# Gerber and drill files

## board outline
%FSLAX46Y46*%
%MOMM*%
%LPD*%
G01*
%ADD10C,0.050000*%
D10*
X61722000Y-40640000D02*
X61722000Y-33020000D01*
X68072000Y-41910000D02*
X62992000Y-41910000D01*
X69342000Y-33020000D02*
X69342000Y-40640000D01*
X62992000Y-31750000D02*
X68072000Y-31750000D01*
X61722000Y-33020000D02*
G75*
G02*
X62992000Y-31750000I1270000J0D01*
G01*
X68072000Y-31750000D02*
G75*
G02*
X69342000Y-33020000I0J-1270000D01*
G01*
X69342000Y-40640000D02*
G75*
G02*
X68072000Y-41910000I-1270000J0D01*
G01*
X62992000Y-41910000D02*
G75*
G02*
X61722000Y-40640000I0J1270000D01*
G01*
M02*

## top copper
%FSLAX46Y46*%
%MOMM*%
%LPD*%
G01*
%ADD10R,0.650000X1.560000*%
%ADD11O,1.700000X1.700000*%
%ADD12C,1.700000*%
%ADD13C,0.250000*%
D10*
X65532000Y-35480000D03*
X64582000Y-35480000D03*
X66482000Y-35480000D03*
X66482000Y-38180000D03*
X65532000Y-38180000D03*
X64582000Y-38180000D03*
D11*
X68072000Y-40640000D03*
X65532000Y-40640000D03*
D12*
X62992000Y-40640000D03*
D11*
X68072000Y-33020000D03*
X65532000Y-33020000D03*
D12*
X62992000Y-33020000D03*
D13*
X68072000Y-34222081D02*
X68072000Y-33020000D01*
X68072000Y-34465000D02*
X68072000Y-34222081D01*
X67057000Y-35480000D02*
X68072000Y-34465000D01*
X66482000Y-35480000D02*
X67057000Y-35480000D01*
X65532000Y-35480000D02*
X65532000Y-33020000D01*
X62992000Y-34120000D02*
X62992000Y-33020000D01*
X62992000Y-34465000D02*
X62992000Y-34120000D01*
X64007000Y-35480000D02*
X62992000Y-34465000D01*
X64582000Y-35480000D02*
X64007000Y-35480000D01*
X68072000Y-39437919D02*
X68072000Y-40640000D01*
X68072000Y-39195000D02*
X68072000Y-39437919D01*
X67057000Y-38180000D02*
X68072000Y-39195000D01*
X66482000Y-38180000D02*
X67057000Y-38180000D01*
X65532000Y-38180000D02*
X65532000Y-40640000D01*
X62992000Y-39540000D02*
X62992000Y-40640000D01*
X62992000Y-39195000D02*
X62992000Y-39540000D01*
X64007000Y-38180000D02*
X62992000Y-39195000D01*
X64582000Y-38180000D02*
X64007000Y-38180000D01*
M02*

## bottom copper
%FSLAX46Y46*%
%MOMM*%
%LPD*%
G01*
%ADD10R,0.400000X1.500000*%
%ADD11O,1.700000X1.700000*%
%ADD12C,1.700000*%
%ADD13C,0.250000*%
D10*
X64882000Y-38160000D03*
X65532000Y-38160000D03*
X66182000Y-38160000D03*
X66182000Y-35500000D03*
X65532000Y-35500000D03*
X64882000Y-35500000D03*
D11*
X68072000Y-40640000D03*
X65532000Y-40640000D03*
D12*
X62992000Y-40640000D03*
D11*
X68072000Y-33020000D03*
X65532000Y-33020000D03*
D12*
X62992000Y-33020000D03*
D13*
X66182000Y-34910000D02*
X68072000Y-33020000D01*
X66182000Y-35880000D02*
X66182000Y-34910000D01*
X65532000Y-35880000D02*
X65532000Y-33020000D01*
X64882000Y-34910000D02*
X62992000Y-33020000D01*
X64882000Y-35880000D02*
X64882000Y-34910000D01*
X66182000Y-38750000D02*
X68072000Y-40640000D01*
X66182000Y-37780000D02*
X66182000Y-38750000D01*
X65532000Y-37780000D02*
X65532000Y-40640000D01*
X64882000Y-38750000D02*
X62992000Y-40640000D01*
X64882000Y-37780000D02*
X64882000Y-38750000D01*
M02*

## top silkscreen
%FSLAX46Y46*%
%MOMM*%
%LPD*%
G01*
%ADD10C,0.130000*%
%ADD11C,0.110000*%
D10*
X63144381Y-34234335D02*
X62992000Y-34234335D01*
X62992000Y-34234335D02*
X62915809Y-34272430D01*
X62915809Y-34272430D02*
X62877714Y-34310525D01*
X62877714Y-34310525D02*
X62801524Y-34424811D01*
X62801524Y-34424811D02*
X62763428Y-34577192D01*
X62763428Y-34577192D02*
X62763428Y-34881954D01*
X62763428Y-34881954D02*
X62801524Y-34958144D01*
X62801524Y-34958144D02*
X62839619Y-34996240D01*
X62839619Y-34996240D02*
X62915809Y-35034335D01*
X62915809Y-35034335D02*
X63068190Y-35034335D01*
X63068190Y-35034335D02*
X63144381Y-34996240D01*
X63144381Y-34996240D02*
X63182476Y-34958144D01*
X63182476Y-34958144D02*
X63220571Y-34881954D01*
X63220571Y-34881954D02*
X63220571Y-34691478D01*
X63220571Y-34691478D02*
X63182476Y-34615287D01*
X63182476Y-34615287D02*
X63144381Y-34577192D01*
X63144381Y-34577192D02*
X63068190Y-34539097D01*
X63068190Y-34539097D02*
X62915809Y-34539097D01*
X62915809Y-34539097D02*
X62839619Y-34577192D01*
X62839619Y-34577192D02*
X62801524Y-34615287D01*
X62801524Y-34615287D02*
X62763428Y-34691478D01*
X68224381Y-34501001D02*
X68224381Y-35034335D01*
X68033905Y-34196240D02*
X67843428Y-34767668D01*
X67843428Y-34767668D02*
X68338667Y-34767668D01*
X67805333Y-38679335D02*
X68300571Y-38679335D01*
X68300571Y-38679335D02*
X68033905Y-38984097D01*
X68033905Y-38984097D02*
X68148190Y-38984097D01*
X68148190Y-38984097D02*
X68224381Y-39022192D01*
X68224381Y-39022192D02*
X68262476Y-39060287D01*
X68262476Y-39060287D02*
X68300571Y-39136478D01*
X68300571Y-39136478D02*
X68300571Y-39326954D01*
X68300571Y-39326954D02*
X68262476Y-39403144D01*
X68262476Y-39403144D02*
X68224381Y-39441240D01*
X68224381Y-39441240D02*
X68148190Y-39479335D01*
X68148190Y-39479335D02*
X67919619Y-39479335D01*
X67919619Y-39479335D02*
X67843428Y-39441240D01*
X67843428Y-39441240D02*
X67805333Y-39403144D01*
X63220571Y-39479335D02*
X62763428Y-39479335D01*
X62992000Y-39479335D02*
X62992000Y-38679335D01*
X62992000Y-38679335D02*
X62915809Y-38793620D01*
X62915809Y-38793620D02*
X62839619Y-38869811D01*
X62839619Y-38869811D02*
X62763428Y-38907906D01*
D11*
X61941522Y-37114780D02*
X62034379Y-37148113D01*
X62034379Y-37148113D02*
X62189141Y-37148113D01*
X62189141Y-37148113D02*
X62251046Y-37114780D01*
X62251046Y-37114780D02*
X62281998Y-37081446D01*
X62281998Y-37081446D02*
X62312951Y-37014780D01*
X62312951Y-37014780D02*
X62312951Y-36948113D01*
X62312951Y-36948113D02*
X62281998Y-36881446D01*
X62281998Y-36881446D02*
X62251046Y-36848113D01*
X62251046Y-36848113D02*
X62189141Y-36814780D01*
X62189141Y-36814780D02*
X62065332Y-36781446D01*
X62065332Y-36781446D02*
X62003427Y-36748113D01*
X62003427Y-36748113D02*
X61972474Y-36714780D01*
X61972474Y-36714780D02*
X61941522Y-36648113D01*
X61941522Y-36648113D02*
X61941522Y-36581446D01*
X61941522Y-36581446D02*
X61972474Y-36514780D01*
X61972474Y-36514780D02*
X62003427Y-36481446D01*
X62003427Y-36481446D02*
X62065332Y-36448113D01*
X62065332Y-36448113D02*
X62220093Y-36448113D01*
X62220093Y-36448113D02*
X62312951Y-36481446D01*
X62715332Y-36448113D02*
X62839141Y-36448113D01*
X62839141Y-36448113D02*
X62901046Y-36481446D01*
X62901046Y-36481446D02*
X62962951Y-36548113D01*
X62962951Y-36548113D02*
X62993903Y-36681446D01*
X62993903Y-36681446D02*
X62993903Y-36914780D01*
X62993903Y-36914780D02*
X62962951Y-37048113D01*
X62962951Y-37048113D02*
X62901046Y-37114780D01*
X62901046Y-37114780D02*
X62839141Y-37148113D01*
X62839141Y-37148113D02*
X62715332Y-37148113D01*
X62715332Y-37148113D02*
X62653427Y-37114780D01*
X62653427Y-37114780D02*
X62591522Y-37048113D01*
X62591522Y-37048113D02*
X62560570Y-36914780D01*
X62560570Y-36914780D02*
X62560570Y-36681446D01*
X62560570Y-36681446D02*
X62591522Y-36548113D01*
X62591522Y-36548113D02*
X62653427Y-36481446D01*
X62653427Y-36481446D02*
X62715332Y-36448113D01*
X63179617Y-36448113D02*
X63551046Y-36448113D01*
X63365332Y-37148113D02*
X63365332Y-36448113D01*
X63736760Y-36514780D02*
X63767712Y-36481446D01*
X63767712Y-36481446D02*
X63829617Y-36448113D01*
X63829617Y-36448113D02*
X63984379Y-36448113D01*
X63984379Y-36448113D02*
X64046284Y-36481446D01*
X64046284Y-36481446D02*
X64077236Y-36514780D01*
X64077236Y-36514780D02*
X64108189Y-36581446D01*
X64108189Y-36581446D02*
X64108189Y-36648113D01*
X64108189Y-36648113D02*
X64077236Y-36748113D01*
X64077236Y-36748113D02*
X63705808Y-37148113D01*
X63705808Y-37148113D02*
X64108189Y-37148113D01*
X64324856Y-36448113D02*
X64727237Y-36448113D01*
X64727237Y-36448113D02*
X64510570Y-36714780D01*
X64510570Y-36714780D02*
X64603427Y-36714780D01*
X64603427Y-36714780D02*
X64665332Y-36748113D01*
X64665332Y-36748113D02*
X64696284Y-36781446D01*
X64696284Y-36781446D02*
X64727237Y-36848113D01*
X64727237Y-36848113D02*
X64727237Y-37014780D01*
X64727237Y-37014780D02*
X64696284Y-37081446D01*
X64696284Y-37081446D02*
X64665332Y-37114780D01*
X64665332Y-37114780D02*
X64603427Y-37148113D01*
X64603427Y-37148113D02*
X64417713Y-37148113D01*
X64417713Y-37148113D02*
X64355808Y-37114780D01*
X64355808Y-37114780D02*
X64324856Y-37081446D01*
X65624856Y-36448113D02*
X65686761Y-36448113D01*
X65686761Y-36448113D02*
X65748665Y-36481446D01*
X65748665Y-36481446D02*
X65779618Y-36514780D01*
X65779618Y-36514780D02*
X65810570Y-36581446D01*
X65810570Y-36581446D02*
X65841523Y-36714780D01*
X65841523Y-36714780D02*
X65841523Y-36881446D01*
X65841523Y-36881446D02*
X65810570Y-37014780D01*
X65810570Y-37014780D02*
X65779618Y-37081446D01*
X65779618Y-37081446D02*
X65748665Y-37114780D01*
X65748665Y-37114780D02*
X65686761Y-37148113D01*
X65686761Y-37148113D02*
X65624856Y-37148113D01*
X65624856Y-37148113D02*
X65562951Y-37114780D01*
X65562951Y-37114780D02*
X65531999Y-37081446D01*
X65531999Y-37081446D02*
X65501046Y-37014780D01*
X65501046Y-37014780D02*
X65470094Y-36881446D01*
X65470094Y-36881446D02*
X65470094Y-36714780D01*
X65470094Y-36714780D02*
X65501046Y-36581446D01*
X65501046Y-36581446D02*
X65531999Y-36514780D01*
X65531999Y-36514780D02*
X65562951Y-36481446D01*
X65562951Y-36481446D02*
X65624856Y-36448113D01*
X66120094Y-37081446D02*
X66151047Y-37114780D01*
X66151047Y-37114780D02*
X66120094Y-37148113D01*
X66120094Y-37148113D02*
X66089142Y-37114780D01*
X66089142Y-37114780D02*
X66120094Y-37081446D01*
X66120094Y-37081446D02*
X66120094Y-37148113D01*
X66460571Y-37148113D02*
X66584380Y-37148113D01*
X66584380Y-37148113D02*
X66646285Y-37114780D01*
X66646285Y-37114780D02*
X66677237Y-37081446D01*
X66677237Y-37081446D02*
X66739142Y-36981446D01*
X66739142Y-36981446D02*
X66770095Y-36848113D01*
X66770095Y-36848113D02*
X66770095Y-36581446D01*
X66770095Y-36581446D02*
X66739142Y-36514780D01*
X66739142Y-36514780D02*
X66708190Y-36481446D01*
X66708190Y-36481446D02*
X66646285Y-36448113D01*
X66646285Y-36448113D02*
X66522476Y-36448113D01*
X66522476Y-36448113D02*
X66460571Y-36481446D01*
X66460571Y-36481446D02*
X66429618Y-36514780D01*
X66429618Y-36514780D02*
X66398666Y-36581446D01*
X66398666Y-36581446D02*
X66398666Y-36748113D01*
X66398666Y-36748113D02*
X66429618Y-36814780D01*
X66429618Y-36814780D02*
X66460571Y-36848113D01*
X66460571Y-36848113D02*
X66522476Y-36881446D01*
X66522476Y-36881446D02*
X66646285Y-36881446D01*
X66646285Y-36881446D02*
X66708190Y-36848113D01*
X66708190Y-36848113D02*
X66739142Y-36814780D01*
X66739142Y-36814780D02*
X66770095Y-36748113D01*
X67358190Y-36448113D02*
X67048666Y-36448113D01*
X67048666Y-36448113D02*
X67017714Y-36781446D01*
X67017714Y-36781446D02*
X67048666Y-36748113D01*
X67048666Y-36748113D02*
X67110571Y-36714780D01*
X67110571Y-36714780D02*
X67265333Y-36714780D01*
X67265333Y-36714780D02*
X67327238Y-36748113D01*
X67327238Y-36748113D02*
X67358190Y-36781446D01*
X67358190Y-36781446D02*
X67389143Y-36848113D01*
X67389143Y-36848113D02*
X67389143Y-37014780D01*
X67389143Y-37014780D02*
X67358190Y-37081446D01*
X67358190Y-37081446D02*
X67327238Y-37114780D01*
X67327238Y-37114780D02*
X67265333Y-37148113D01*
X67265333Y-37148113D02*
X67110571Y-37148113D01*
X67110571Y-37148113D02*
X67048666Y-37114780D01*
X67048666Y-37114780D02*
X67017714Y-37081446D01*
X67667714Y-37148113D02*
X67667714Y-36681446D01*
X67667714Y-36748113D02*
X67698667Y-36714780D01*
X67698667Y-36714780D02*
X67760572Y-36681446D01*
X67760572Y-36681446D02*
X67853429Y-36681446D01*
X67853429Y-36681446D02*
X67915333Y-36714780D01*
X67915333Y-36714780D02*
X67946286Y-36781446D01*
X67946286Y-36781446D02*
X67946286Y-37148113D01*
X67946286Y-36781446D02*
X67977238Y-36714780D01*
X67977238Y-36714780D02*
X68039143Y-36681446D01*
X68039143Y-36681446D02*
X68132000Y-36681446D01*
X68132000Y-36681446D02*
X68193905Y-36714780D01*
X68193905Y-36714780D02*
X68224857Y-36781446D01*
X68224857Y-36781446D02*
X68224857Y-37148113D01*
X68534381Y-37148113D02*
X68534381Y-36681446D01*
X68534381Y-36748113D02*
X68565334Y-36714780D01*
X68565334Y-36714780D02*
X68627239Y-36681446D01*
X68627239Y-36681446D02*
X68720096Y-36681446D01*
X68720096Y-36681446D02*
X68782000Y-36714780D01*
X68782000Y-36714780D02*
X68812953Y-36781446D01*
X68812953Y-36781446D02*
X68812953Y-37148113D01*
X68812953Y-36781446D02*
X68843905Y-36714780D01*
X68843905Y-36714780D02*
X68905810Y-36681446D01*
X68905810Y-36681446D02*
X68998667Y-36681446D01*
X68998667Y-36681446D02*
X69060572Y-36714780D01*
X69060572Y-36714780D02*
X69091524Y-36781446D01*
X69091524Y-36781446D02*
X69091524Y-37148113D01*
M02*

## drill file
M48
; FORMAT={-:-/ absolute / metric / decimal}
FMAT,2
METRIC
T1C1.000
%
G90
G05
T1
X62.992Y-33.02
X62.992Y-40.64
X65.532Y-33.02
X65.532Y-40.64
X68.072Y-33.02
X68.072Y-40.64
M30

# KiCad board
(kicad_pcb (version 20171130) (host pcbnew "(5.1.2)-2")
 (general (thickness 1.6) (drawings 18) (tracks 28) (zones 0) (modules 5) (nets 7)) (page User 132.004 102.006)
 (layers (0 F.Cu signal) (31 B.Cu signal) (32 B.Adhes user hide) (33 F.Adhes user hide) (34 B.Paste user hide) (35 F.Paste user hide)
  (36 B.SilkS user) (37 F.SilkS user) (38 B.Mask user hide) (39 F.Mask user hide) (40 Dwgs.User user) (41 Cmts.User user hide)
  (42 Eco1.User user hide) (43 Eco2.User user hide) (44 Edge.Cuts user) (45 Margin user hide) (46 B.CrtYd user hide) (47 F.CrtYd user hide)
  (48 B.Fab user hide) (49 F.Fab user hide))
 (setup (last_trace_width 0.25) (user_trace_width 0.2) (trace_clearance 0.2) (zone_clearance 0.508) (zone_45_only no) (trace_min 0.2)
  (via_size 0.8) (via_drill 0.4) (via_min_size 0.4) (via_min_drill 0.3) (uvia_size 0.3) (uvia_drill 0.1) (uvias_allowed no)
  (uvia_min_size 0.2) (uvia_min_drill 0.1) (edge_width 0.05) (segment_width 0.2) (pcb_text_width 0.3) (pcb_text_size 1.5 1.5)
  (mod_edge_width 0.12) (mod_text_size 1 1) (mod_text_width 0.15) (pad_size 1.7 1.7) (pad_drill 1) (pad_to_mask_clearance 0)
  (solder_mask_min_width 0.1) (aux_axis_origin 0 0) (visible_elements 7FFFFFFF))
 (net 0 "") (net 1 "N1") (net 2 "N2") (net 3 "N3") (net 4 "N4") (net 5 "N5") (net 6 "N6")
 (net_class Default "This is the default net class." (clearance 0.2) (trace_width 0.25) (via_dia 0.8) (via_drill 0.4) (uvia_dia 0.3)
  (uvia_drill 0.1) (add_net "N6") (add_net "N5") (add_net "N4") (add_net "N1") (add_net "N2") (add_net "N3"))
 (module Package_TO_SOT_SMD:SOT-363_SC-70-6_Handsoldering (layer B.Cu) (at 65.532 36.83 270)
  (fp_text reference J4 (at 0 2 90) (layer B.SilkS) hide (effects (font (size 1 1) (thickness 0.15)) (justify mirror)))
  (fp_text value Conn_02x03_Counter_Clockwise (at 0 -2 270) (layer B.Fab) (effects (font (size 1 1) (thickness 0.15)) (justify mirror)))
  (pad 6 smd rect (at 1.33 0.65 270) (size 1.5 0.4) (layers B.Cu B.Paste B.Mask) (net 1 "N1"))
  (pad 5 smd rect (at 1.33 0 270) (size 1.5 0.4) (layers B.Cu B.Paste B.Mask) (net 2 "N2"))
  (pad 4 smd rect (at 1.33 -0.65 270) (size 1.5 0.4) (layers B.Cu B.Paste B.Mask) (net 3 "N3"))
  (pad 3 smd rect (at -1.33 -0.65 270) (size 1.5 0.4) (layers B.Cu B.Paste B.Mask) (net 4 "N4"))
  (pad 2 smd rect (at -1.33 0 270) (size 1.5 0.4) (layers B.Cu B.Paste B.Mask) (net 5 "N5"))
  (pad 1 smd rect (at -1.33 0.65 270) (size 1.5 0.4) (layers B.Cu B.Paste B.Mask) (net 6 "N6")))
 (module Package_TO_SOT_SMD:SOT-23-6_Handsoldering (layer F.Cu) (at 65.532 36.83 90)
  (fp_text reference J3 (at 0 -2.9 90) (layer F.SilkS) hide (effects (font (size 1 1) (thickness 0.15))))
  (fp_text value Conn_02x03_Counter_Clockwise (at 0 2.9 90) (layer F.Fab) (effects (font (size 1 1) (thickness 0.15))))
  (pad 5 smd rect (at 1.35 0 90) (size 1.56 0.65) (layers F.Cu F.Paste F.Mask) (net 5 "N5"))
  (pad 6 smd rect (at 1.35 -0.95 90) (size 1.56 0.65) (layers F.Cu F.Paste F.Mask) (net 6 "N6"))
  (pad 4 smd rect (at 1.35 0.95 90) (size 1.56 0.65) (layers F.Cu F.Paste F.Mask) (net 4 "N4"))
  (pad 3 smd rect (at -1.35 0.95 90) (size 1.56 0.65) (layers F.Cu F.Paste F.Mask) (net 3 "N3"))
  (pad 2 smd rect (at -1.35 0 90) (size 1.56 0.65) (layers F.Cu F.Paste F.Mask) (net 2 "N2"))
  (pad 1 smd rect (at -1.35 -0.95 90) (size 1.56 0.65) (layers F.Cu F.Paste F.Mask) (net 1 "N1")))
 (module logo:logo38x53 (layer B.Cu) (at 62.992 36.8046 180)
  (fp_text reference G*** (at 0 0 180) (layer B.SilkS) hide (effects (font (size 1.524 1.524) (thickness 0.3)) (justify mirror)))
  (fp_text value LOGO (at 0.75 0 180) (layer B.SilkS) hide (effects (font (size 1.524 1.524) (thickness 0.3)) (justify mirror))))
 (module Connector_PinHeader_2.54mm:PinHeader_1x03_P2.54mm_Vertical (layer F.Cu) (at 62.992 40.64 90)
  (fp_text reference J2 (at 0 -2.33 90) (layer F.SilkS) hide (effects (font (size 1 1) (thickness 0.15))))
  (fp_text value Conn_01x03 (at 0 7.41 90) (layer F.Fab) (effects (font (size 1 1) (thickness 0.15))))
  (pad 3 thru_hole oval (at 0 5.08 90) (size 1.7 1.7) (drill 1) (layers *.Cu *.Mask) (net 3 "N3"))
  (pad 2 thru_hole oval (at 0 2.54 90) (size 1.7 1.7) (drill 1) (layers *.Cu *.Mask) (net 2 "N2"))
  (pad 1 thru_hole circle (at 0 0 90) (size 1.7 1.7) (drill 1) (layers *.Cu *.Mask) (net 1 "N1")))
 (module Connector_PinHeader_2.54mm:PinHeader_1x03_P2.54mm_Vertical (layer F.Cu) (at 62.992 33.02 90)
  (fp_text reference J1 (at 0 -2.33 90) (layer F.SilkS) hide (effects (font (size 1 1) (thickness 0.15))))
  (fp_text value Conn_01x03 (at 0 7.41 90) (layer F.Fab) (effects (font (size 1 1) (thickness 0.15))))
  (pad 3 thru_hole oval (at 0 5.08 90) (size 1.7 1.7) (drill 1) (layers *.Cu *.Mask) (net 4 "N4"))
  (pad 2 thru_hole oval (at 0 2.54 90) (size 1.7 1.7) (drill 1) (layers *.Cu *.Mask) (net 5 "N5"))
  (pad 1 thru_hole circle (at 0 0 90) (size 1.7 1.7) (drill 1) (layers *.Cu *.Mask) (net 6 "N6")))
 (gr_line (start 61.722 40.64) (end 61.722 33.02) (layer Edge.Cuts) (width 0.05))
 (gr_line (start 68.072 41.91) (end 62.992 41.91) (layer Edge.Cuts) (width 0.05))
 (gr_line (start 69.342 33.02) (end 69.342 40.64) (layer Edge.Cuts) (width 0.05))
 (gr_line (start 62.992 31.75) (end 68.072 31.75) (layer Edge.Cuts) (width 0.05))
 (gr_arc (start 62.992 33.02) (end 62.992 31.75) (angle -90) (layer Edge.Cuts) (width 0.05))
 (gr_arc (start 68.072 33.02) (end 69.342 33.02) (angle -90) (layer Edge.Cuts) (width 0.05))
 (gr_arc (start 68.072 40.64) (end 68.072 41.91) (angle -90) (layer Edge.Cuts) (width 0.05))
 (gr_arc (start 62.992 40.64) (end 61.722 40.64) (angle -90) (layer Edge.Cuts) (width 0.05))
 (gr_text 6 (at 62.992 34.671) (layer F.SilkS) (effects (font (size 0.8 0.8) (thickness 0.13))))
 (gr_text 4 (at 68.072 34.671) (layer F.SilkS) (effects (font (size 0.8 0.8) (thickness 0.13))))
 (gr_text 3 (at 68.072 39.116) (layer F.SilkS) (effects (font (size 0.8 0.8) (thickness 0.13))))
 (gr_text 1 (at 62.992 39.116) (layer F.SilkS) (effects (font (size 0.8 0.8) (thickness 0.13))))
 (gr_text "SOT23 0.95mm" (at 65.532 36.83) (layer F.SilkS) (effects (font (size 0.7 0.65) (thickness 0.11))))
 (segment (start 68.072 34.222081) (end 68.072 33.02) (width 0.25) (layer F.Cu) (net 4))
 (segment (start 68.072 34.465) (end 68.072 34.222081) (width 0.25) (layer F.Cu) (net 4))
 (segment (start 67.057 35.48) (end 68.072 34.465) (width 0.25) (layer F.Cu) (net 4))
 (segment (start 66.482 35.48) (end 67.057 35.48) (width 0.25) (layer F.Cu) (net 4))
 (segment (start 66.182 34.91) (end 68.072 33.02) (width 0.25) (layer B.Cu) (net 4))
 (segment (start 66.182 35.88) (end 66.182 34.91) (width 0.25) (layer B.Cu) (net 4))
 (segment (start 65.532 35.48) (end 65.532 33.02) (width 0.25) (layer F.Cu) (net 5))
 (segment (start 65.532 35.88) (end 65.532 33.02) (width 0.25) (layer B.Cu) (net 5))
 (segment (start 62.992 34.12) (end 62.992 33.02) (width 0.25) (layer F.Cu) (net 6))
 (segment (start 62.992 34.465) (end 62.992 34.12) (width 0.25) (layer F.Cu) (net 6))
 (segment (start 64.007 35.48) (end 62.992 34.465) (width 0.25) (layer F.Cu) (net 6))
 (segment (start 64.582 35.48) (end 64.007 35.48) (width 0.25) (layer F.Cu) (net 6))
 (segment (start 64.882 34.91) (end 62.992 33.02) (width 0.25) (layer B.Cu) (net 6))
 (segment (start 64.882 35.88) (end 64.882 34.91) (width 0.25) (layer B.Cu) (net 6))
 (segment (start 68.072 39.437919) (end 68.072 40.64) (width 0.25) (layer F.Cu) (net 3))
 (segment (start 68.072 39.195) (end 68.072 39.437919) (width 0.25) (layer F.Cu) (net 3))
 (segment (start 67.057 38.18) (end 68.072 39.195) (width 0.25) (layer F.Cu) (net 3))
 (segment (start 66.482 38.18) (end 67.057 38.18) (width 0.25) (layer F.Cu) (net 3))
 (segment (start 66.182 38.75) (end 68.072 40.64) (width 0.25) (layer B.Cu) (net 3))
 (segment (start 66.182 37.78) (end 66.182 38.75) (width 0.25) (layer B.Cu) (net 3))
 (segment (start 65.532 38.18) (end 65.532 40.64) (width 0.25) (layer F.Cu) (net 2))
 (segment (start 65.532 37.78) (end 65.532 40.64) (width 0.25) (layer B.Cu) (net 2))
 (segment (start 62.992 39.54) (end 62.992 40.64) (width 0.25) (layer F.Cu) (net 1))
 (segment (start 62.992 39.195) (end 62.992 39.54) (width 0.25) (layer F.Cu) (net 1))
 (segment (start 64.007 38.18) (end 62.992 39.195) (width 0.25) (layer F.Cu) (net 1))
 (segment (start 64.582 38.18) (end 64.007 38.18) (width 0.25) (layer F.Cu) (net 1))
 (segment (start 64.882 38.75) (end 62.992 40.64) (width 0.25) (layer B.Cu) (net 1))
 (segment (start 64.882 37.78) (end 64.882 38.75) (width 0.25) (layer B.Cu) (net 1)))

